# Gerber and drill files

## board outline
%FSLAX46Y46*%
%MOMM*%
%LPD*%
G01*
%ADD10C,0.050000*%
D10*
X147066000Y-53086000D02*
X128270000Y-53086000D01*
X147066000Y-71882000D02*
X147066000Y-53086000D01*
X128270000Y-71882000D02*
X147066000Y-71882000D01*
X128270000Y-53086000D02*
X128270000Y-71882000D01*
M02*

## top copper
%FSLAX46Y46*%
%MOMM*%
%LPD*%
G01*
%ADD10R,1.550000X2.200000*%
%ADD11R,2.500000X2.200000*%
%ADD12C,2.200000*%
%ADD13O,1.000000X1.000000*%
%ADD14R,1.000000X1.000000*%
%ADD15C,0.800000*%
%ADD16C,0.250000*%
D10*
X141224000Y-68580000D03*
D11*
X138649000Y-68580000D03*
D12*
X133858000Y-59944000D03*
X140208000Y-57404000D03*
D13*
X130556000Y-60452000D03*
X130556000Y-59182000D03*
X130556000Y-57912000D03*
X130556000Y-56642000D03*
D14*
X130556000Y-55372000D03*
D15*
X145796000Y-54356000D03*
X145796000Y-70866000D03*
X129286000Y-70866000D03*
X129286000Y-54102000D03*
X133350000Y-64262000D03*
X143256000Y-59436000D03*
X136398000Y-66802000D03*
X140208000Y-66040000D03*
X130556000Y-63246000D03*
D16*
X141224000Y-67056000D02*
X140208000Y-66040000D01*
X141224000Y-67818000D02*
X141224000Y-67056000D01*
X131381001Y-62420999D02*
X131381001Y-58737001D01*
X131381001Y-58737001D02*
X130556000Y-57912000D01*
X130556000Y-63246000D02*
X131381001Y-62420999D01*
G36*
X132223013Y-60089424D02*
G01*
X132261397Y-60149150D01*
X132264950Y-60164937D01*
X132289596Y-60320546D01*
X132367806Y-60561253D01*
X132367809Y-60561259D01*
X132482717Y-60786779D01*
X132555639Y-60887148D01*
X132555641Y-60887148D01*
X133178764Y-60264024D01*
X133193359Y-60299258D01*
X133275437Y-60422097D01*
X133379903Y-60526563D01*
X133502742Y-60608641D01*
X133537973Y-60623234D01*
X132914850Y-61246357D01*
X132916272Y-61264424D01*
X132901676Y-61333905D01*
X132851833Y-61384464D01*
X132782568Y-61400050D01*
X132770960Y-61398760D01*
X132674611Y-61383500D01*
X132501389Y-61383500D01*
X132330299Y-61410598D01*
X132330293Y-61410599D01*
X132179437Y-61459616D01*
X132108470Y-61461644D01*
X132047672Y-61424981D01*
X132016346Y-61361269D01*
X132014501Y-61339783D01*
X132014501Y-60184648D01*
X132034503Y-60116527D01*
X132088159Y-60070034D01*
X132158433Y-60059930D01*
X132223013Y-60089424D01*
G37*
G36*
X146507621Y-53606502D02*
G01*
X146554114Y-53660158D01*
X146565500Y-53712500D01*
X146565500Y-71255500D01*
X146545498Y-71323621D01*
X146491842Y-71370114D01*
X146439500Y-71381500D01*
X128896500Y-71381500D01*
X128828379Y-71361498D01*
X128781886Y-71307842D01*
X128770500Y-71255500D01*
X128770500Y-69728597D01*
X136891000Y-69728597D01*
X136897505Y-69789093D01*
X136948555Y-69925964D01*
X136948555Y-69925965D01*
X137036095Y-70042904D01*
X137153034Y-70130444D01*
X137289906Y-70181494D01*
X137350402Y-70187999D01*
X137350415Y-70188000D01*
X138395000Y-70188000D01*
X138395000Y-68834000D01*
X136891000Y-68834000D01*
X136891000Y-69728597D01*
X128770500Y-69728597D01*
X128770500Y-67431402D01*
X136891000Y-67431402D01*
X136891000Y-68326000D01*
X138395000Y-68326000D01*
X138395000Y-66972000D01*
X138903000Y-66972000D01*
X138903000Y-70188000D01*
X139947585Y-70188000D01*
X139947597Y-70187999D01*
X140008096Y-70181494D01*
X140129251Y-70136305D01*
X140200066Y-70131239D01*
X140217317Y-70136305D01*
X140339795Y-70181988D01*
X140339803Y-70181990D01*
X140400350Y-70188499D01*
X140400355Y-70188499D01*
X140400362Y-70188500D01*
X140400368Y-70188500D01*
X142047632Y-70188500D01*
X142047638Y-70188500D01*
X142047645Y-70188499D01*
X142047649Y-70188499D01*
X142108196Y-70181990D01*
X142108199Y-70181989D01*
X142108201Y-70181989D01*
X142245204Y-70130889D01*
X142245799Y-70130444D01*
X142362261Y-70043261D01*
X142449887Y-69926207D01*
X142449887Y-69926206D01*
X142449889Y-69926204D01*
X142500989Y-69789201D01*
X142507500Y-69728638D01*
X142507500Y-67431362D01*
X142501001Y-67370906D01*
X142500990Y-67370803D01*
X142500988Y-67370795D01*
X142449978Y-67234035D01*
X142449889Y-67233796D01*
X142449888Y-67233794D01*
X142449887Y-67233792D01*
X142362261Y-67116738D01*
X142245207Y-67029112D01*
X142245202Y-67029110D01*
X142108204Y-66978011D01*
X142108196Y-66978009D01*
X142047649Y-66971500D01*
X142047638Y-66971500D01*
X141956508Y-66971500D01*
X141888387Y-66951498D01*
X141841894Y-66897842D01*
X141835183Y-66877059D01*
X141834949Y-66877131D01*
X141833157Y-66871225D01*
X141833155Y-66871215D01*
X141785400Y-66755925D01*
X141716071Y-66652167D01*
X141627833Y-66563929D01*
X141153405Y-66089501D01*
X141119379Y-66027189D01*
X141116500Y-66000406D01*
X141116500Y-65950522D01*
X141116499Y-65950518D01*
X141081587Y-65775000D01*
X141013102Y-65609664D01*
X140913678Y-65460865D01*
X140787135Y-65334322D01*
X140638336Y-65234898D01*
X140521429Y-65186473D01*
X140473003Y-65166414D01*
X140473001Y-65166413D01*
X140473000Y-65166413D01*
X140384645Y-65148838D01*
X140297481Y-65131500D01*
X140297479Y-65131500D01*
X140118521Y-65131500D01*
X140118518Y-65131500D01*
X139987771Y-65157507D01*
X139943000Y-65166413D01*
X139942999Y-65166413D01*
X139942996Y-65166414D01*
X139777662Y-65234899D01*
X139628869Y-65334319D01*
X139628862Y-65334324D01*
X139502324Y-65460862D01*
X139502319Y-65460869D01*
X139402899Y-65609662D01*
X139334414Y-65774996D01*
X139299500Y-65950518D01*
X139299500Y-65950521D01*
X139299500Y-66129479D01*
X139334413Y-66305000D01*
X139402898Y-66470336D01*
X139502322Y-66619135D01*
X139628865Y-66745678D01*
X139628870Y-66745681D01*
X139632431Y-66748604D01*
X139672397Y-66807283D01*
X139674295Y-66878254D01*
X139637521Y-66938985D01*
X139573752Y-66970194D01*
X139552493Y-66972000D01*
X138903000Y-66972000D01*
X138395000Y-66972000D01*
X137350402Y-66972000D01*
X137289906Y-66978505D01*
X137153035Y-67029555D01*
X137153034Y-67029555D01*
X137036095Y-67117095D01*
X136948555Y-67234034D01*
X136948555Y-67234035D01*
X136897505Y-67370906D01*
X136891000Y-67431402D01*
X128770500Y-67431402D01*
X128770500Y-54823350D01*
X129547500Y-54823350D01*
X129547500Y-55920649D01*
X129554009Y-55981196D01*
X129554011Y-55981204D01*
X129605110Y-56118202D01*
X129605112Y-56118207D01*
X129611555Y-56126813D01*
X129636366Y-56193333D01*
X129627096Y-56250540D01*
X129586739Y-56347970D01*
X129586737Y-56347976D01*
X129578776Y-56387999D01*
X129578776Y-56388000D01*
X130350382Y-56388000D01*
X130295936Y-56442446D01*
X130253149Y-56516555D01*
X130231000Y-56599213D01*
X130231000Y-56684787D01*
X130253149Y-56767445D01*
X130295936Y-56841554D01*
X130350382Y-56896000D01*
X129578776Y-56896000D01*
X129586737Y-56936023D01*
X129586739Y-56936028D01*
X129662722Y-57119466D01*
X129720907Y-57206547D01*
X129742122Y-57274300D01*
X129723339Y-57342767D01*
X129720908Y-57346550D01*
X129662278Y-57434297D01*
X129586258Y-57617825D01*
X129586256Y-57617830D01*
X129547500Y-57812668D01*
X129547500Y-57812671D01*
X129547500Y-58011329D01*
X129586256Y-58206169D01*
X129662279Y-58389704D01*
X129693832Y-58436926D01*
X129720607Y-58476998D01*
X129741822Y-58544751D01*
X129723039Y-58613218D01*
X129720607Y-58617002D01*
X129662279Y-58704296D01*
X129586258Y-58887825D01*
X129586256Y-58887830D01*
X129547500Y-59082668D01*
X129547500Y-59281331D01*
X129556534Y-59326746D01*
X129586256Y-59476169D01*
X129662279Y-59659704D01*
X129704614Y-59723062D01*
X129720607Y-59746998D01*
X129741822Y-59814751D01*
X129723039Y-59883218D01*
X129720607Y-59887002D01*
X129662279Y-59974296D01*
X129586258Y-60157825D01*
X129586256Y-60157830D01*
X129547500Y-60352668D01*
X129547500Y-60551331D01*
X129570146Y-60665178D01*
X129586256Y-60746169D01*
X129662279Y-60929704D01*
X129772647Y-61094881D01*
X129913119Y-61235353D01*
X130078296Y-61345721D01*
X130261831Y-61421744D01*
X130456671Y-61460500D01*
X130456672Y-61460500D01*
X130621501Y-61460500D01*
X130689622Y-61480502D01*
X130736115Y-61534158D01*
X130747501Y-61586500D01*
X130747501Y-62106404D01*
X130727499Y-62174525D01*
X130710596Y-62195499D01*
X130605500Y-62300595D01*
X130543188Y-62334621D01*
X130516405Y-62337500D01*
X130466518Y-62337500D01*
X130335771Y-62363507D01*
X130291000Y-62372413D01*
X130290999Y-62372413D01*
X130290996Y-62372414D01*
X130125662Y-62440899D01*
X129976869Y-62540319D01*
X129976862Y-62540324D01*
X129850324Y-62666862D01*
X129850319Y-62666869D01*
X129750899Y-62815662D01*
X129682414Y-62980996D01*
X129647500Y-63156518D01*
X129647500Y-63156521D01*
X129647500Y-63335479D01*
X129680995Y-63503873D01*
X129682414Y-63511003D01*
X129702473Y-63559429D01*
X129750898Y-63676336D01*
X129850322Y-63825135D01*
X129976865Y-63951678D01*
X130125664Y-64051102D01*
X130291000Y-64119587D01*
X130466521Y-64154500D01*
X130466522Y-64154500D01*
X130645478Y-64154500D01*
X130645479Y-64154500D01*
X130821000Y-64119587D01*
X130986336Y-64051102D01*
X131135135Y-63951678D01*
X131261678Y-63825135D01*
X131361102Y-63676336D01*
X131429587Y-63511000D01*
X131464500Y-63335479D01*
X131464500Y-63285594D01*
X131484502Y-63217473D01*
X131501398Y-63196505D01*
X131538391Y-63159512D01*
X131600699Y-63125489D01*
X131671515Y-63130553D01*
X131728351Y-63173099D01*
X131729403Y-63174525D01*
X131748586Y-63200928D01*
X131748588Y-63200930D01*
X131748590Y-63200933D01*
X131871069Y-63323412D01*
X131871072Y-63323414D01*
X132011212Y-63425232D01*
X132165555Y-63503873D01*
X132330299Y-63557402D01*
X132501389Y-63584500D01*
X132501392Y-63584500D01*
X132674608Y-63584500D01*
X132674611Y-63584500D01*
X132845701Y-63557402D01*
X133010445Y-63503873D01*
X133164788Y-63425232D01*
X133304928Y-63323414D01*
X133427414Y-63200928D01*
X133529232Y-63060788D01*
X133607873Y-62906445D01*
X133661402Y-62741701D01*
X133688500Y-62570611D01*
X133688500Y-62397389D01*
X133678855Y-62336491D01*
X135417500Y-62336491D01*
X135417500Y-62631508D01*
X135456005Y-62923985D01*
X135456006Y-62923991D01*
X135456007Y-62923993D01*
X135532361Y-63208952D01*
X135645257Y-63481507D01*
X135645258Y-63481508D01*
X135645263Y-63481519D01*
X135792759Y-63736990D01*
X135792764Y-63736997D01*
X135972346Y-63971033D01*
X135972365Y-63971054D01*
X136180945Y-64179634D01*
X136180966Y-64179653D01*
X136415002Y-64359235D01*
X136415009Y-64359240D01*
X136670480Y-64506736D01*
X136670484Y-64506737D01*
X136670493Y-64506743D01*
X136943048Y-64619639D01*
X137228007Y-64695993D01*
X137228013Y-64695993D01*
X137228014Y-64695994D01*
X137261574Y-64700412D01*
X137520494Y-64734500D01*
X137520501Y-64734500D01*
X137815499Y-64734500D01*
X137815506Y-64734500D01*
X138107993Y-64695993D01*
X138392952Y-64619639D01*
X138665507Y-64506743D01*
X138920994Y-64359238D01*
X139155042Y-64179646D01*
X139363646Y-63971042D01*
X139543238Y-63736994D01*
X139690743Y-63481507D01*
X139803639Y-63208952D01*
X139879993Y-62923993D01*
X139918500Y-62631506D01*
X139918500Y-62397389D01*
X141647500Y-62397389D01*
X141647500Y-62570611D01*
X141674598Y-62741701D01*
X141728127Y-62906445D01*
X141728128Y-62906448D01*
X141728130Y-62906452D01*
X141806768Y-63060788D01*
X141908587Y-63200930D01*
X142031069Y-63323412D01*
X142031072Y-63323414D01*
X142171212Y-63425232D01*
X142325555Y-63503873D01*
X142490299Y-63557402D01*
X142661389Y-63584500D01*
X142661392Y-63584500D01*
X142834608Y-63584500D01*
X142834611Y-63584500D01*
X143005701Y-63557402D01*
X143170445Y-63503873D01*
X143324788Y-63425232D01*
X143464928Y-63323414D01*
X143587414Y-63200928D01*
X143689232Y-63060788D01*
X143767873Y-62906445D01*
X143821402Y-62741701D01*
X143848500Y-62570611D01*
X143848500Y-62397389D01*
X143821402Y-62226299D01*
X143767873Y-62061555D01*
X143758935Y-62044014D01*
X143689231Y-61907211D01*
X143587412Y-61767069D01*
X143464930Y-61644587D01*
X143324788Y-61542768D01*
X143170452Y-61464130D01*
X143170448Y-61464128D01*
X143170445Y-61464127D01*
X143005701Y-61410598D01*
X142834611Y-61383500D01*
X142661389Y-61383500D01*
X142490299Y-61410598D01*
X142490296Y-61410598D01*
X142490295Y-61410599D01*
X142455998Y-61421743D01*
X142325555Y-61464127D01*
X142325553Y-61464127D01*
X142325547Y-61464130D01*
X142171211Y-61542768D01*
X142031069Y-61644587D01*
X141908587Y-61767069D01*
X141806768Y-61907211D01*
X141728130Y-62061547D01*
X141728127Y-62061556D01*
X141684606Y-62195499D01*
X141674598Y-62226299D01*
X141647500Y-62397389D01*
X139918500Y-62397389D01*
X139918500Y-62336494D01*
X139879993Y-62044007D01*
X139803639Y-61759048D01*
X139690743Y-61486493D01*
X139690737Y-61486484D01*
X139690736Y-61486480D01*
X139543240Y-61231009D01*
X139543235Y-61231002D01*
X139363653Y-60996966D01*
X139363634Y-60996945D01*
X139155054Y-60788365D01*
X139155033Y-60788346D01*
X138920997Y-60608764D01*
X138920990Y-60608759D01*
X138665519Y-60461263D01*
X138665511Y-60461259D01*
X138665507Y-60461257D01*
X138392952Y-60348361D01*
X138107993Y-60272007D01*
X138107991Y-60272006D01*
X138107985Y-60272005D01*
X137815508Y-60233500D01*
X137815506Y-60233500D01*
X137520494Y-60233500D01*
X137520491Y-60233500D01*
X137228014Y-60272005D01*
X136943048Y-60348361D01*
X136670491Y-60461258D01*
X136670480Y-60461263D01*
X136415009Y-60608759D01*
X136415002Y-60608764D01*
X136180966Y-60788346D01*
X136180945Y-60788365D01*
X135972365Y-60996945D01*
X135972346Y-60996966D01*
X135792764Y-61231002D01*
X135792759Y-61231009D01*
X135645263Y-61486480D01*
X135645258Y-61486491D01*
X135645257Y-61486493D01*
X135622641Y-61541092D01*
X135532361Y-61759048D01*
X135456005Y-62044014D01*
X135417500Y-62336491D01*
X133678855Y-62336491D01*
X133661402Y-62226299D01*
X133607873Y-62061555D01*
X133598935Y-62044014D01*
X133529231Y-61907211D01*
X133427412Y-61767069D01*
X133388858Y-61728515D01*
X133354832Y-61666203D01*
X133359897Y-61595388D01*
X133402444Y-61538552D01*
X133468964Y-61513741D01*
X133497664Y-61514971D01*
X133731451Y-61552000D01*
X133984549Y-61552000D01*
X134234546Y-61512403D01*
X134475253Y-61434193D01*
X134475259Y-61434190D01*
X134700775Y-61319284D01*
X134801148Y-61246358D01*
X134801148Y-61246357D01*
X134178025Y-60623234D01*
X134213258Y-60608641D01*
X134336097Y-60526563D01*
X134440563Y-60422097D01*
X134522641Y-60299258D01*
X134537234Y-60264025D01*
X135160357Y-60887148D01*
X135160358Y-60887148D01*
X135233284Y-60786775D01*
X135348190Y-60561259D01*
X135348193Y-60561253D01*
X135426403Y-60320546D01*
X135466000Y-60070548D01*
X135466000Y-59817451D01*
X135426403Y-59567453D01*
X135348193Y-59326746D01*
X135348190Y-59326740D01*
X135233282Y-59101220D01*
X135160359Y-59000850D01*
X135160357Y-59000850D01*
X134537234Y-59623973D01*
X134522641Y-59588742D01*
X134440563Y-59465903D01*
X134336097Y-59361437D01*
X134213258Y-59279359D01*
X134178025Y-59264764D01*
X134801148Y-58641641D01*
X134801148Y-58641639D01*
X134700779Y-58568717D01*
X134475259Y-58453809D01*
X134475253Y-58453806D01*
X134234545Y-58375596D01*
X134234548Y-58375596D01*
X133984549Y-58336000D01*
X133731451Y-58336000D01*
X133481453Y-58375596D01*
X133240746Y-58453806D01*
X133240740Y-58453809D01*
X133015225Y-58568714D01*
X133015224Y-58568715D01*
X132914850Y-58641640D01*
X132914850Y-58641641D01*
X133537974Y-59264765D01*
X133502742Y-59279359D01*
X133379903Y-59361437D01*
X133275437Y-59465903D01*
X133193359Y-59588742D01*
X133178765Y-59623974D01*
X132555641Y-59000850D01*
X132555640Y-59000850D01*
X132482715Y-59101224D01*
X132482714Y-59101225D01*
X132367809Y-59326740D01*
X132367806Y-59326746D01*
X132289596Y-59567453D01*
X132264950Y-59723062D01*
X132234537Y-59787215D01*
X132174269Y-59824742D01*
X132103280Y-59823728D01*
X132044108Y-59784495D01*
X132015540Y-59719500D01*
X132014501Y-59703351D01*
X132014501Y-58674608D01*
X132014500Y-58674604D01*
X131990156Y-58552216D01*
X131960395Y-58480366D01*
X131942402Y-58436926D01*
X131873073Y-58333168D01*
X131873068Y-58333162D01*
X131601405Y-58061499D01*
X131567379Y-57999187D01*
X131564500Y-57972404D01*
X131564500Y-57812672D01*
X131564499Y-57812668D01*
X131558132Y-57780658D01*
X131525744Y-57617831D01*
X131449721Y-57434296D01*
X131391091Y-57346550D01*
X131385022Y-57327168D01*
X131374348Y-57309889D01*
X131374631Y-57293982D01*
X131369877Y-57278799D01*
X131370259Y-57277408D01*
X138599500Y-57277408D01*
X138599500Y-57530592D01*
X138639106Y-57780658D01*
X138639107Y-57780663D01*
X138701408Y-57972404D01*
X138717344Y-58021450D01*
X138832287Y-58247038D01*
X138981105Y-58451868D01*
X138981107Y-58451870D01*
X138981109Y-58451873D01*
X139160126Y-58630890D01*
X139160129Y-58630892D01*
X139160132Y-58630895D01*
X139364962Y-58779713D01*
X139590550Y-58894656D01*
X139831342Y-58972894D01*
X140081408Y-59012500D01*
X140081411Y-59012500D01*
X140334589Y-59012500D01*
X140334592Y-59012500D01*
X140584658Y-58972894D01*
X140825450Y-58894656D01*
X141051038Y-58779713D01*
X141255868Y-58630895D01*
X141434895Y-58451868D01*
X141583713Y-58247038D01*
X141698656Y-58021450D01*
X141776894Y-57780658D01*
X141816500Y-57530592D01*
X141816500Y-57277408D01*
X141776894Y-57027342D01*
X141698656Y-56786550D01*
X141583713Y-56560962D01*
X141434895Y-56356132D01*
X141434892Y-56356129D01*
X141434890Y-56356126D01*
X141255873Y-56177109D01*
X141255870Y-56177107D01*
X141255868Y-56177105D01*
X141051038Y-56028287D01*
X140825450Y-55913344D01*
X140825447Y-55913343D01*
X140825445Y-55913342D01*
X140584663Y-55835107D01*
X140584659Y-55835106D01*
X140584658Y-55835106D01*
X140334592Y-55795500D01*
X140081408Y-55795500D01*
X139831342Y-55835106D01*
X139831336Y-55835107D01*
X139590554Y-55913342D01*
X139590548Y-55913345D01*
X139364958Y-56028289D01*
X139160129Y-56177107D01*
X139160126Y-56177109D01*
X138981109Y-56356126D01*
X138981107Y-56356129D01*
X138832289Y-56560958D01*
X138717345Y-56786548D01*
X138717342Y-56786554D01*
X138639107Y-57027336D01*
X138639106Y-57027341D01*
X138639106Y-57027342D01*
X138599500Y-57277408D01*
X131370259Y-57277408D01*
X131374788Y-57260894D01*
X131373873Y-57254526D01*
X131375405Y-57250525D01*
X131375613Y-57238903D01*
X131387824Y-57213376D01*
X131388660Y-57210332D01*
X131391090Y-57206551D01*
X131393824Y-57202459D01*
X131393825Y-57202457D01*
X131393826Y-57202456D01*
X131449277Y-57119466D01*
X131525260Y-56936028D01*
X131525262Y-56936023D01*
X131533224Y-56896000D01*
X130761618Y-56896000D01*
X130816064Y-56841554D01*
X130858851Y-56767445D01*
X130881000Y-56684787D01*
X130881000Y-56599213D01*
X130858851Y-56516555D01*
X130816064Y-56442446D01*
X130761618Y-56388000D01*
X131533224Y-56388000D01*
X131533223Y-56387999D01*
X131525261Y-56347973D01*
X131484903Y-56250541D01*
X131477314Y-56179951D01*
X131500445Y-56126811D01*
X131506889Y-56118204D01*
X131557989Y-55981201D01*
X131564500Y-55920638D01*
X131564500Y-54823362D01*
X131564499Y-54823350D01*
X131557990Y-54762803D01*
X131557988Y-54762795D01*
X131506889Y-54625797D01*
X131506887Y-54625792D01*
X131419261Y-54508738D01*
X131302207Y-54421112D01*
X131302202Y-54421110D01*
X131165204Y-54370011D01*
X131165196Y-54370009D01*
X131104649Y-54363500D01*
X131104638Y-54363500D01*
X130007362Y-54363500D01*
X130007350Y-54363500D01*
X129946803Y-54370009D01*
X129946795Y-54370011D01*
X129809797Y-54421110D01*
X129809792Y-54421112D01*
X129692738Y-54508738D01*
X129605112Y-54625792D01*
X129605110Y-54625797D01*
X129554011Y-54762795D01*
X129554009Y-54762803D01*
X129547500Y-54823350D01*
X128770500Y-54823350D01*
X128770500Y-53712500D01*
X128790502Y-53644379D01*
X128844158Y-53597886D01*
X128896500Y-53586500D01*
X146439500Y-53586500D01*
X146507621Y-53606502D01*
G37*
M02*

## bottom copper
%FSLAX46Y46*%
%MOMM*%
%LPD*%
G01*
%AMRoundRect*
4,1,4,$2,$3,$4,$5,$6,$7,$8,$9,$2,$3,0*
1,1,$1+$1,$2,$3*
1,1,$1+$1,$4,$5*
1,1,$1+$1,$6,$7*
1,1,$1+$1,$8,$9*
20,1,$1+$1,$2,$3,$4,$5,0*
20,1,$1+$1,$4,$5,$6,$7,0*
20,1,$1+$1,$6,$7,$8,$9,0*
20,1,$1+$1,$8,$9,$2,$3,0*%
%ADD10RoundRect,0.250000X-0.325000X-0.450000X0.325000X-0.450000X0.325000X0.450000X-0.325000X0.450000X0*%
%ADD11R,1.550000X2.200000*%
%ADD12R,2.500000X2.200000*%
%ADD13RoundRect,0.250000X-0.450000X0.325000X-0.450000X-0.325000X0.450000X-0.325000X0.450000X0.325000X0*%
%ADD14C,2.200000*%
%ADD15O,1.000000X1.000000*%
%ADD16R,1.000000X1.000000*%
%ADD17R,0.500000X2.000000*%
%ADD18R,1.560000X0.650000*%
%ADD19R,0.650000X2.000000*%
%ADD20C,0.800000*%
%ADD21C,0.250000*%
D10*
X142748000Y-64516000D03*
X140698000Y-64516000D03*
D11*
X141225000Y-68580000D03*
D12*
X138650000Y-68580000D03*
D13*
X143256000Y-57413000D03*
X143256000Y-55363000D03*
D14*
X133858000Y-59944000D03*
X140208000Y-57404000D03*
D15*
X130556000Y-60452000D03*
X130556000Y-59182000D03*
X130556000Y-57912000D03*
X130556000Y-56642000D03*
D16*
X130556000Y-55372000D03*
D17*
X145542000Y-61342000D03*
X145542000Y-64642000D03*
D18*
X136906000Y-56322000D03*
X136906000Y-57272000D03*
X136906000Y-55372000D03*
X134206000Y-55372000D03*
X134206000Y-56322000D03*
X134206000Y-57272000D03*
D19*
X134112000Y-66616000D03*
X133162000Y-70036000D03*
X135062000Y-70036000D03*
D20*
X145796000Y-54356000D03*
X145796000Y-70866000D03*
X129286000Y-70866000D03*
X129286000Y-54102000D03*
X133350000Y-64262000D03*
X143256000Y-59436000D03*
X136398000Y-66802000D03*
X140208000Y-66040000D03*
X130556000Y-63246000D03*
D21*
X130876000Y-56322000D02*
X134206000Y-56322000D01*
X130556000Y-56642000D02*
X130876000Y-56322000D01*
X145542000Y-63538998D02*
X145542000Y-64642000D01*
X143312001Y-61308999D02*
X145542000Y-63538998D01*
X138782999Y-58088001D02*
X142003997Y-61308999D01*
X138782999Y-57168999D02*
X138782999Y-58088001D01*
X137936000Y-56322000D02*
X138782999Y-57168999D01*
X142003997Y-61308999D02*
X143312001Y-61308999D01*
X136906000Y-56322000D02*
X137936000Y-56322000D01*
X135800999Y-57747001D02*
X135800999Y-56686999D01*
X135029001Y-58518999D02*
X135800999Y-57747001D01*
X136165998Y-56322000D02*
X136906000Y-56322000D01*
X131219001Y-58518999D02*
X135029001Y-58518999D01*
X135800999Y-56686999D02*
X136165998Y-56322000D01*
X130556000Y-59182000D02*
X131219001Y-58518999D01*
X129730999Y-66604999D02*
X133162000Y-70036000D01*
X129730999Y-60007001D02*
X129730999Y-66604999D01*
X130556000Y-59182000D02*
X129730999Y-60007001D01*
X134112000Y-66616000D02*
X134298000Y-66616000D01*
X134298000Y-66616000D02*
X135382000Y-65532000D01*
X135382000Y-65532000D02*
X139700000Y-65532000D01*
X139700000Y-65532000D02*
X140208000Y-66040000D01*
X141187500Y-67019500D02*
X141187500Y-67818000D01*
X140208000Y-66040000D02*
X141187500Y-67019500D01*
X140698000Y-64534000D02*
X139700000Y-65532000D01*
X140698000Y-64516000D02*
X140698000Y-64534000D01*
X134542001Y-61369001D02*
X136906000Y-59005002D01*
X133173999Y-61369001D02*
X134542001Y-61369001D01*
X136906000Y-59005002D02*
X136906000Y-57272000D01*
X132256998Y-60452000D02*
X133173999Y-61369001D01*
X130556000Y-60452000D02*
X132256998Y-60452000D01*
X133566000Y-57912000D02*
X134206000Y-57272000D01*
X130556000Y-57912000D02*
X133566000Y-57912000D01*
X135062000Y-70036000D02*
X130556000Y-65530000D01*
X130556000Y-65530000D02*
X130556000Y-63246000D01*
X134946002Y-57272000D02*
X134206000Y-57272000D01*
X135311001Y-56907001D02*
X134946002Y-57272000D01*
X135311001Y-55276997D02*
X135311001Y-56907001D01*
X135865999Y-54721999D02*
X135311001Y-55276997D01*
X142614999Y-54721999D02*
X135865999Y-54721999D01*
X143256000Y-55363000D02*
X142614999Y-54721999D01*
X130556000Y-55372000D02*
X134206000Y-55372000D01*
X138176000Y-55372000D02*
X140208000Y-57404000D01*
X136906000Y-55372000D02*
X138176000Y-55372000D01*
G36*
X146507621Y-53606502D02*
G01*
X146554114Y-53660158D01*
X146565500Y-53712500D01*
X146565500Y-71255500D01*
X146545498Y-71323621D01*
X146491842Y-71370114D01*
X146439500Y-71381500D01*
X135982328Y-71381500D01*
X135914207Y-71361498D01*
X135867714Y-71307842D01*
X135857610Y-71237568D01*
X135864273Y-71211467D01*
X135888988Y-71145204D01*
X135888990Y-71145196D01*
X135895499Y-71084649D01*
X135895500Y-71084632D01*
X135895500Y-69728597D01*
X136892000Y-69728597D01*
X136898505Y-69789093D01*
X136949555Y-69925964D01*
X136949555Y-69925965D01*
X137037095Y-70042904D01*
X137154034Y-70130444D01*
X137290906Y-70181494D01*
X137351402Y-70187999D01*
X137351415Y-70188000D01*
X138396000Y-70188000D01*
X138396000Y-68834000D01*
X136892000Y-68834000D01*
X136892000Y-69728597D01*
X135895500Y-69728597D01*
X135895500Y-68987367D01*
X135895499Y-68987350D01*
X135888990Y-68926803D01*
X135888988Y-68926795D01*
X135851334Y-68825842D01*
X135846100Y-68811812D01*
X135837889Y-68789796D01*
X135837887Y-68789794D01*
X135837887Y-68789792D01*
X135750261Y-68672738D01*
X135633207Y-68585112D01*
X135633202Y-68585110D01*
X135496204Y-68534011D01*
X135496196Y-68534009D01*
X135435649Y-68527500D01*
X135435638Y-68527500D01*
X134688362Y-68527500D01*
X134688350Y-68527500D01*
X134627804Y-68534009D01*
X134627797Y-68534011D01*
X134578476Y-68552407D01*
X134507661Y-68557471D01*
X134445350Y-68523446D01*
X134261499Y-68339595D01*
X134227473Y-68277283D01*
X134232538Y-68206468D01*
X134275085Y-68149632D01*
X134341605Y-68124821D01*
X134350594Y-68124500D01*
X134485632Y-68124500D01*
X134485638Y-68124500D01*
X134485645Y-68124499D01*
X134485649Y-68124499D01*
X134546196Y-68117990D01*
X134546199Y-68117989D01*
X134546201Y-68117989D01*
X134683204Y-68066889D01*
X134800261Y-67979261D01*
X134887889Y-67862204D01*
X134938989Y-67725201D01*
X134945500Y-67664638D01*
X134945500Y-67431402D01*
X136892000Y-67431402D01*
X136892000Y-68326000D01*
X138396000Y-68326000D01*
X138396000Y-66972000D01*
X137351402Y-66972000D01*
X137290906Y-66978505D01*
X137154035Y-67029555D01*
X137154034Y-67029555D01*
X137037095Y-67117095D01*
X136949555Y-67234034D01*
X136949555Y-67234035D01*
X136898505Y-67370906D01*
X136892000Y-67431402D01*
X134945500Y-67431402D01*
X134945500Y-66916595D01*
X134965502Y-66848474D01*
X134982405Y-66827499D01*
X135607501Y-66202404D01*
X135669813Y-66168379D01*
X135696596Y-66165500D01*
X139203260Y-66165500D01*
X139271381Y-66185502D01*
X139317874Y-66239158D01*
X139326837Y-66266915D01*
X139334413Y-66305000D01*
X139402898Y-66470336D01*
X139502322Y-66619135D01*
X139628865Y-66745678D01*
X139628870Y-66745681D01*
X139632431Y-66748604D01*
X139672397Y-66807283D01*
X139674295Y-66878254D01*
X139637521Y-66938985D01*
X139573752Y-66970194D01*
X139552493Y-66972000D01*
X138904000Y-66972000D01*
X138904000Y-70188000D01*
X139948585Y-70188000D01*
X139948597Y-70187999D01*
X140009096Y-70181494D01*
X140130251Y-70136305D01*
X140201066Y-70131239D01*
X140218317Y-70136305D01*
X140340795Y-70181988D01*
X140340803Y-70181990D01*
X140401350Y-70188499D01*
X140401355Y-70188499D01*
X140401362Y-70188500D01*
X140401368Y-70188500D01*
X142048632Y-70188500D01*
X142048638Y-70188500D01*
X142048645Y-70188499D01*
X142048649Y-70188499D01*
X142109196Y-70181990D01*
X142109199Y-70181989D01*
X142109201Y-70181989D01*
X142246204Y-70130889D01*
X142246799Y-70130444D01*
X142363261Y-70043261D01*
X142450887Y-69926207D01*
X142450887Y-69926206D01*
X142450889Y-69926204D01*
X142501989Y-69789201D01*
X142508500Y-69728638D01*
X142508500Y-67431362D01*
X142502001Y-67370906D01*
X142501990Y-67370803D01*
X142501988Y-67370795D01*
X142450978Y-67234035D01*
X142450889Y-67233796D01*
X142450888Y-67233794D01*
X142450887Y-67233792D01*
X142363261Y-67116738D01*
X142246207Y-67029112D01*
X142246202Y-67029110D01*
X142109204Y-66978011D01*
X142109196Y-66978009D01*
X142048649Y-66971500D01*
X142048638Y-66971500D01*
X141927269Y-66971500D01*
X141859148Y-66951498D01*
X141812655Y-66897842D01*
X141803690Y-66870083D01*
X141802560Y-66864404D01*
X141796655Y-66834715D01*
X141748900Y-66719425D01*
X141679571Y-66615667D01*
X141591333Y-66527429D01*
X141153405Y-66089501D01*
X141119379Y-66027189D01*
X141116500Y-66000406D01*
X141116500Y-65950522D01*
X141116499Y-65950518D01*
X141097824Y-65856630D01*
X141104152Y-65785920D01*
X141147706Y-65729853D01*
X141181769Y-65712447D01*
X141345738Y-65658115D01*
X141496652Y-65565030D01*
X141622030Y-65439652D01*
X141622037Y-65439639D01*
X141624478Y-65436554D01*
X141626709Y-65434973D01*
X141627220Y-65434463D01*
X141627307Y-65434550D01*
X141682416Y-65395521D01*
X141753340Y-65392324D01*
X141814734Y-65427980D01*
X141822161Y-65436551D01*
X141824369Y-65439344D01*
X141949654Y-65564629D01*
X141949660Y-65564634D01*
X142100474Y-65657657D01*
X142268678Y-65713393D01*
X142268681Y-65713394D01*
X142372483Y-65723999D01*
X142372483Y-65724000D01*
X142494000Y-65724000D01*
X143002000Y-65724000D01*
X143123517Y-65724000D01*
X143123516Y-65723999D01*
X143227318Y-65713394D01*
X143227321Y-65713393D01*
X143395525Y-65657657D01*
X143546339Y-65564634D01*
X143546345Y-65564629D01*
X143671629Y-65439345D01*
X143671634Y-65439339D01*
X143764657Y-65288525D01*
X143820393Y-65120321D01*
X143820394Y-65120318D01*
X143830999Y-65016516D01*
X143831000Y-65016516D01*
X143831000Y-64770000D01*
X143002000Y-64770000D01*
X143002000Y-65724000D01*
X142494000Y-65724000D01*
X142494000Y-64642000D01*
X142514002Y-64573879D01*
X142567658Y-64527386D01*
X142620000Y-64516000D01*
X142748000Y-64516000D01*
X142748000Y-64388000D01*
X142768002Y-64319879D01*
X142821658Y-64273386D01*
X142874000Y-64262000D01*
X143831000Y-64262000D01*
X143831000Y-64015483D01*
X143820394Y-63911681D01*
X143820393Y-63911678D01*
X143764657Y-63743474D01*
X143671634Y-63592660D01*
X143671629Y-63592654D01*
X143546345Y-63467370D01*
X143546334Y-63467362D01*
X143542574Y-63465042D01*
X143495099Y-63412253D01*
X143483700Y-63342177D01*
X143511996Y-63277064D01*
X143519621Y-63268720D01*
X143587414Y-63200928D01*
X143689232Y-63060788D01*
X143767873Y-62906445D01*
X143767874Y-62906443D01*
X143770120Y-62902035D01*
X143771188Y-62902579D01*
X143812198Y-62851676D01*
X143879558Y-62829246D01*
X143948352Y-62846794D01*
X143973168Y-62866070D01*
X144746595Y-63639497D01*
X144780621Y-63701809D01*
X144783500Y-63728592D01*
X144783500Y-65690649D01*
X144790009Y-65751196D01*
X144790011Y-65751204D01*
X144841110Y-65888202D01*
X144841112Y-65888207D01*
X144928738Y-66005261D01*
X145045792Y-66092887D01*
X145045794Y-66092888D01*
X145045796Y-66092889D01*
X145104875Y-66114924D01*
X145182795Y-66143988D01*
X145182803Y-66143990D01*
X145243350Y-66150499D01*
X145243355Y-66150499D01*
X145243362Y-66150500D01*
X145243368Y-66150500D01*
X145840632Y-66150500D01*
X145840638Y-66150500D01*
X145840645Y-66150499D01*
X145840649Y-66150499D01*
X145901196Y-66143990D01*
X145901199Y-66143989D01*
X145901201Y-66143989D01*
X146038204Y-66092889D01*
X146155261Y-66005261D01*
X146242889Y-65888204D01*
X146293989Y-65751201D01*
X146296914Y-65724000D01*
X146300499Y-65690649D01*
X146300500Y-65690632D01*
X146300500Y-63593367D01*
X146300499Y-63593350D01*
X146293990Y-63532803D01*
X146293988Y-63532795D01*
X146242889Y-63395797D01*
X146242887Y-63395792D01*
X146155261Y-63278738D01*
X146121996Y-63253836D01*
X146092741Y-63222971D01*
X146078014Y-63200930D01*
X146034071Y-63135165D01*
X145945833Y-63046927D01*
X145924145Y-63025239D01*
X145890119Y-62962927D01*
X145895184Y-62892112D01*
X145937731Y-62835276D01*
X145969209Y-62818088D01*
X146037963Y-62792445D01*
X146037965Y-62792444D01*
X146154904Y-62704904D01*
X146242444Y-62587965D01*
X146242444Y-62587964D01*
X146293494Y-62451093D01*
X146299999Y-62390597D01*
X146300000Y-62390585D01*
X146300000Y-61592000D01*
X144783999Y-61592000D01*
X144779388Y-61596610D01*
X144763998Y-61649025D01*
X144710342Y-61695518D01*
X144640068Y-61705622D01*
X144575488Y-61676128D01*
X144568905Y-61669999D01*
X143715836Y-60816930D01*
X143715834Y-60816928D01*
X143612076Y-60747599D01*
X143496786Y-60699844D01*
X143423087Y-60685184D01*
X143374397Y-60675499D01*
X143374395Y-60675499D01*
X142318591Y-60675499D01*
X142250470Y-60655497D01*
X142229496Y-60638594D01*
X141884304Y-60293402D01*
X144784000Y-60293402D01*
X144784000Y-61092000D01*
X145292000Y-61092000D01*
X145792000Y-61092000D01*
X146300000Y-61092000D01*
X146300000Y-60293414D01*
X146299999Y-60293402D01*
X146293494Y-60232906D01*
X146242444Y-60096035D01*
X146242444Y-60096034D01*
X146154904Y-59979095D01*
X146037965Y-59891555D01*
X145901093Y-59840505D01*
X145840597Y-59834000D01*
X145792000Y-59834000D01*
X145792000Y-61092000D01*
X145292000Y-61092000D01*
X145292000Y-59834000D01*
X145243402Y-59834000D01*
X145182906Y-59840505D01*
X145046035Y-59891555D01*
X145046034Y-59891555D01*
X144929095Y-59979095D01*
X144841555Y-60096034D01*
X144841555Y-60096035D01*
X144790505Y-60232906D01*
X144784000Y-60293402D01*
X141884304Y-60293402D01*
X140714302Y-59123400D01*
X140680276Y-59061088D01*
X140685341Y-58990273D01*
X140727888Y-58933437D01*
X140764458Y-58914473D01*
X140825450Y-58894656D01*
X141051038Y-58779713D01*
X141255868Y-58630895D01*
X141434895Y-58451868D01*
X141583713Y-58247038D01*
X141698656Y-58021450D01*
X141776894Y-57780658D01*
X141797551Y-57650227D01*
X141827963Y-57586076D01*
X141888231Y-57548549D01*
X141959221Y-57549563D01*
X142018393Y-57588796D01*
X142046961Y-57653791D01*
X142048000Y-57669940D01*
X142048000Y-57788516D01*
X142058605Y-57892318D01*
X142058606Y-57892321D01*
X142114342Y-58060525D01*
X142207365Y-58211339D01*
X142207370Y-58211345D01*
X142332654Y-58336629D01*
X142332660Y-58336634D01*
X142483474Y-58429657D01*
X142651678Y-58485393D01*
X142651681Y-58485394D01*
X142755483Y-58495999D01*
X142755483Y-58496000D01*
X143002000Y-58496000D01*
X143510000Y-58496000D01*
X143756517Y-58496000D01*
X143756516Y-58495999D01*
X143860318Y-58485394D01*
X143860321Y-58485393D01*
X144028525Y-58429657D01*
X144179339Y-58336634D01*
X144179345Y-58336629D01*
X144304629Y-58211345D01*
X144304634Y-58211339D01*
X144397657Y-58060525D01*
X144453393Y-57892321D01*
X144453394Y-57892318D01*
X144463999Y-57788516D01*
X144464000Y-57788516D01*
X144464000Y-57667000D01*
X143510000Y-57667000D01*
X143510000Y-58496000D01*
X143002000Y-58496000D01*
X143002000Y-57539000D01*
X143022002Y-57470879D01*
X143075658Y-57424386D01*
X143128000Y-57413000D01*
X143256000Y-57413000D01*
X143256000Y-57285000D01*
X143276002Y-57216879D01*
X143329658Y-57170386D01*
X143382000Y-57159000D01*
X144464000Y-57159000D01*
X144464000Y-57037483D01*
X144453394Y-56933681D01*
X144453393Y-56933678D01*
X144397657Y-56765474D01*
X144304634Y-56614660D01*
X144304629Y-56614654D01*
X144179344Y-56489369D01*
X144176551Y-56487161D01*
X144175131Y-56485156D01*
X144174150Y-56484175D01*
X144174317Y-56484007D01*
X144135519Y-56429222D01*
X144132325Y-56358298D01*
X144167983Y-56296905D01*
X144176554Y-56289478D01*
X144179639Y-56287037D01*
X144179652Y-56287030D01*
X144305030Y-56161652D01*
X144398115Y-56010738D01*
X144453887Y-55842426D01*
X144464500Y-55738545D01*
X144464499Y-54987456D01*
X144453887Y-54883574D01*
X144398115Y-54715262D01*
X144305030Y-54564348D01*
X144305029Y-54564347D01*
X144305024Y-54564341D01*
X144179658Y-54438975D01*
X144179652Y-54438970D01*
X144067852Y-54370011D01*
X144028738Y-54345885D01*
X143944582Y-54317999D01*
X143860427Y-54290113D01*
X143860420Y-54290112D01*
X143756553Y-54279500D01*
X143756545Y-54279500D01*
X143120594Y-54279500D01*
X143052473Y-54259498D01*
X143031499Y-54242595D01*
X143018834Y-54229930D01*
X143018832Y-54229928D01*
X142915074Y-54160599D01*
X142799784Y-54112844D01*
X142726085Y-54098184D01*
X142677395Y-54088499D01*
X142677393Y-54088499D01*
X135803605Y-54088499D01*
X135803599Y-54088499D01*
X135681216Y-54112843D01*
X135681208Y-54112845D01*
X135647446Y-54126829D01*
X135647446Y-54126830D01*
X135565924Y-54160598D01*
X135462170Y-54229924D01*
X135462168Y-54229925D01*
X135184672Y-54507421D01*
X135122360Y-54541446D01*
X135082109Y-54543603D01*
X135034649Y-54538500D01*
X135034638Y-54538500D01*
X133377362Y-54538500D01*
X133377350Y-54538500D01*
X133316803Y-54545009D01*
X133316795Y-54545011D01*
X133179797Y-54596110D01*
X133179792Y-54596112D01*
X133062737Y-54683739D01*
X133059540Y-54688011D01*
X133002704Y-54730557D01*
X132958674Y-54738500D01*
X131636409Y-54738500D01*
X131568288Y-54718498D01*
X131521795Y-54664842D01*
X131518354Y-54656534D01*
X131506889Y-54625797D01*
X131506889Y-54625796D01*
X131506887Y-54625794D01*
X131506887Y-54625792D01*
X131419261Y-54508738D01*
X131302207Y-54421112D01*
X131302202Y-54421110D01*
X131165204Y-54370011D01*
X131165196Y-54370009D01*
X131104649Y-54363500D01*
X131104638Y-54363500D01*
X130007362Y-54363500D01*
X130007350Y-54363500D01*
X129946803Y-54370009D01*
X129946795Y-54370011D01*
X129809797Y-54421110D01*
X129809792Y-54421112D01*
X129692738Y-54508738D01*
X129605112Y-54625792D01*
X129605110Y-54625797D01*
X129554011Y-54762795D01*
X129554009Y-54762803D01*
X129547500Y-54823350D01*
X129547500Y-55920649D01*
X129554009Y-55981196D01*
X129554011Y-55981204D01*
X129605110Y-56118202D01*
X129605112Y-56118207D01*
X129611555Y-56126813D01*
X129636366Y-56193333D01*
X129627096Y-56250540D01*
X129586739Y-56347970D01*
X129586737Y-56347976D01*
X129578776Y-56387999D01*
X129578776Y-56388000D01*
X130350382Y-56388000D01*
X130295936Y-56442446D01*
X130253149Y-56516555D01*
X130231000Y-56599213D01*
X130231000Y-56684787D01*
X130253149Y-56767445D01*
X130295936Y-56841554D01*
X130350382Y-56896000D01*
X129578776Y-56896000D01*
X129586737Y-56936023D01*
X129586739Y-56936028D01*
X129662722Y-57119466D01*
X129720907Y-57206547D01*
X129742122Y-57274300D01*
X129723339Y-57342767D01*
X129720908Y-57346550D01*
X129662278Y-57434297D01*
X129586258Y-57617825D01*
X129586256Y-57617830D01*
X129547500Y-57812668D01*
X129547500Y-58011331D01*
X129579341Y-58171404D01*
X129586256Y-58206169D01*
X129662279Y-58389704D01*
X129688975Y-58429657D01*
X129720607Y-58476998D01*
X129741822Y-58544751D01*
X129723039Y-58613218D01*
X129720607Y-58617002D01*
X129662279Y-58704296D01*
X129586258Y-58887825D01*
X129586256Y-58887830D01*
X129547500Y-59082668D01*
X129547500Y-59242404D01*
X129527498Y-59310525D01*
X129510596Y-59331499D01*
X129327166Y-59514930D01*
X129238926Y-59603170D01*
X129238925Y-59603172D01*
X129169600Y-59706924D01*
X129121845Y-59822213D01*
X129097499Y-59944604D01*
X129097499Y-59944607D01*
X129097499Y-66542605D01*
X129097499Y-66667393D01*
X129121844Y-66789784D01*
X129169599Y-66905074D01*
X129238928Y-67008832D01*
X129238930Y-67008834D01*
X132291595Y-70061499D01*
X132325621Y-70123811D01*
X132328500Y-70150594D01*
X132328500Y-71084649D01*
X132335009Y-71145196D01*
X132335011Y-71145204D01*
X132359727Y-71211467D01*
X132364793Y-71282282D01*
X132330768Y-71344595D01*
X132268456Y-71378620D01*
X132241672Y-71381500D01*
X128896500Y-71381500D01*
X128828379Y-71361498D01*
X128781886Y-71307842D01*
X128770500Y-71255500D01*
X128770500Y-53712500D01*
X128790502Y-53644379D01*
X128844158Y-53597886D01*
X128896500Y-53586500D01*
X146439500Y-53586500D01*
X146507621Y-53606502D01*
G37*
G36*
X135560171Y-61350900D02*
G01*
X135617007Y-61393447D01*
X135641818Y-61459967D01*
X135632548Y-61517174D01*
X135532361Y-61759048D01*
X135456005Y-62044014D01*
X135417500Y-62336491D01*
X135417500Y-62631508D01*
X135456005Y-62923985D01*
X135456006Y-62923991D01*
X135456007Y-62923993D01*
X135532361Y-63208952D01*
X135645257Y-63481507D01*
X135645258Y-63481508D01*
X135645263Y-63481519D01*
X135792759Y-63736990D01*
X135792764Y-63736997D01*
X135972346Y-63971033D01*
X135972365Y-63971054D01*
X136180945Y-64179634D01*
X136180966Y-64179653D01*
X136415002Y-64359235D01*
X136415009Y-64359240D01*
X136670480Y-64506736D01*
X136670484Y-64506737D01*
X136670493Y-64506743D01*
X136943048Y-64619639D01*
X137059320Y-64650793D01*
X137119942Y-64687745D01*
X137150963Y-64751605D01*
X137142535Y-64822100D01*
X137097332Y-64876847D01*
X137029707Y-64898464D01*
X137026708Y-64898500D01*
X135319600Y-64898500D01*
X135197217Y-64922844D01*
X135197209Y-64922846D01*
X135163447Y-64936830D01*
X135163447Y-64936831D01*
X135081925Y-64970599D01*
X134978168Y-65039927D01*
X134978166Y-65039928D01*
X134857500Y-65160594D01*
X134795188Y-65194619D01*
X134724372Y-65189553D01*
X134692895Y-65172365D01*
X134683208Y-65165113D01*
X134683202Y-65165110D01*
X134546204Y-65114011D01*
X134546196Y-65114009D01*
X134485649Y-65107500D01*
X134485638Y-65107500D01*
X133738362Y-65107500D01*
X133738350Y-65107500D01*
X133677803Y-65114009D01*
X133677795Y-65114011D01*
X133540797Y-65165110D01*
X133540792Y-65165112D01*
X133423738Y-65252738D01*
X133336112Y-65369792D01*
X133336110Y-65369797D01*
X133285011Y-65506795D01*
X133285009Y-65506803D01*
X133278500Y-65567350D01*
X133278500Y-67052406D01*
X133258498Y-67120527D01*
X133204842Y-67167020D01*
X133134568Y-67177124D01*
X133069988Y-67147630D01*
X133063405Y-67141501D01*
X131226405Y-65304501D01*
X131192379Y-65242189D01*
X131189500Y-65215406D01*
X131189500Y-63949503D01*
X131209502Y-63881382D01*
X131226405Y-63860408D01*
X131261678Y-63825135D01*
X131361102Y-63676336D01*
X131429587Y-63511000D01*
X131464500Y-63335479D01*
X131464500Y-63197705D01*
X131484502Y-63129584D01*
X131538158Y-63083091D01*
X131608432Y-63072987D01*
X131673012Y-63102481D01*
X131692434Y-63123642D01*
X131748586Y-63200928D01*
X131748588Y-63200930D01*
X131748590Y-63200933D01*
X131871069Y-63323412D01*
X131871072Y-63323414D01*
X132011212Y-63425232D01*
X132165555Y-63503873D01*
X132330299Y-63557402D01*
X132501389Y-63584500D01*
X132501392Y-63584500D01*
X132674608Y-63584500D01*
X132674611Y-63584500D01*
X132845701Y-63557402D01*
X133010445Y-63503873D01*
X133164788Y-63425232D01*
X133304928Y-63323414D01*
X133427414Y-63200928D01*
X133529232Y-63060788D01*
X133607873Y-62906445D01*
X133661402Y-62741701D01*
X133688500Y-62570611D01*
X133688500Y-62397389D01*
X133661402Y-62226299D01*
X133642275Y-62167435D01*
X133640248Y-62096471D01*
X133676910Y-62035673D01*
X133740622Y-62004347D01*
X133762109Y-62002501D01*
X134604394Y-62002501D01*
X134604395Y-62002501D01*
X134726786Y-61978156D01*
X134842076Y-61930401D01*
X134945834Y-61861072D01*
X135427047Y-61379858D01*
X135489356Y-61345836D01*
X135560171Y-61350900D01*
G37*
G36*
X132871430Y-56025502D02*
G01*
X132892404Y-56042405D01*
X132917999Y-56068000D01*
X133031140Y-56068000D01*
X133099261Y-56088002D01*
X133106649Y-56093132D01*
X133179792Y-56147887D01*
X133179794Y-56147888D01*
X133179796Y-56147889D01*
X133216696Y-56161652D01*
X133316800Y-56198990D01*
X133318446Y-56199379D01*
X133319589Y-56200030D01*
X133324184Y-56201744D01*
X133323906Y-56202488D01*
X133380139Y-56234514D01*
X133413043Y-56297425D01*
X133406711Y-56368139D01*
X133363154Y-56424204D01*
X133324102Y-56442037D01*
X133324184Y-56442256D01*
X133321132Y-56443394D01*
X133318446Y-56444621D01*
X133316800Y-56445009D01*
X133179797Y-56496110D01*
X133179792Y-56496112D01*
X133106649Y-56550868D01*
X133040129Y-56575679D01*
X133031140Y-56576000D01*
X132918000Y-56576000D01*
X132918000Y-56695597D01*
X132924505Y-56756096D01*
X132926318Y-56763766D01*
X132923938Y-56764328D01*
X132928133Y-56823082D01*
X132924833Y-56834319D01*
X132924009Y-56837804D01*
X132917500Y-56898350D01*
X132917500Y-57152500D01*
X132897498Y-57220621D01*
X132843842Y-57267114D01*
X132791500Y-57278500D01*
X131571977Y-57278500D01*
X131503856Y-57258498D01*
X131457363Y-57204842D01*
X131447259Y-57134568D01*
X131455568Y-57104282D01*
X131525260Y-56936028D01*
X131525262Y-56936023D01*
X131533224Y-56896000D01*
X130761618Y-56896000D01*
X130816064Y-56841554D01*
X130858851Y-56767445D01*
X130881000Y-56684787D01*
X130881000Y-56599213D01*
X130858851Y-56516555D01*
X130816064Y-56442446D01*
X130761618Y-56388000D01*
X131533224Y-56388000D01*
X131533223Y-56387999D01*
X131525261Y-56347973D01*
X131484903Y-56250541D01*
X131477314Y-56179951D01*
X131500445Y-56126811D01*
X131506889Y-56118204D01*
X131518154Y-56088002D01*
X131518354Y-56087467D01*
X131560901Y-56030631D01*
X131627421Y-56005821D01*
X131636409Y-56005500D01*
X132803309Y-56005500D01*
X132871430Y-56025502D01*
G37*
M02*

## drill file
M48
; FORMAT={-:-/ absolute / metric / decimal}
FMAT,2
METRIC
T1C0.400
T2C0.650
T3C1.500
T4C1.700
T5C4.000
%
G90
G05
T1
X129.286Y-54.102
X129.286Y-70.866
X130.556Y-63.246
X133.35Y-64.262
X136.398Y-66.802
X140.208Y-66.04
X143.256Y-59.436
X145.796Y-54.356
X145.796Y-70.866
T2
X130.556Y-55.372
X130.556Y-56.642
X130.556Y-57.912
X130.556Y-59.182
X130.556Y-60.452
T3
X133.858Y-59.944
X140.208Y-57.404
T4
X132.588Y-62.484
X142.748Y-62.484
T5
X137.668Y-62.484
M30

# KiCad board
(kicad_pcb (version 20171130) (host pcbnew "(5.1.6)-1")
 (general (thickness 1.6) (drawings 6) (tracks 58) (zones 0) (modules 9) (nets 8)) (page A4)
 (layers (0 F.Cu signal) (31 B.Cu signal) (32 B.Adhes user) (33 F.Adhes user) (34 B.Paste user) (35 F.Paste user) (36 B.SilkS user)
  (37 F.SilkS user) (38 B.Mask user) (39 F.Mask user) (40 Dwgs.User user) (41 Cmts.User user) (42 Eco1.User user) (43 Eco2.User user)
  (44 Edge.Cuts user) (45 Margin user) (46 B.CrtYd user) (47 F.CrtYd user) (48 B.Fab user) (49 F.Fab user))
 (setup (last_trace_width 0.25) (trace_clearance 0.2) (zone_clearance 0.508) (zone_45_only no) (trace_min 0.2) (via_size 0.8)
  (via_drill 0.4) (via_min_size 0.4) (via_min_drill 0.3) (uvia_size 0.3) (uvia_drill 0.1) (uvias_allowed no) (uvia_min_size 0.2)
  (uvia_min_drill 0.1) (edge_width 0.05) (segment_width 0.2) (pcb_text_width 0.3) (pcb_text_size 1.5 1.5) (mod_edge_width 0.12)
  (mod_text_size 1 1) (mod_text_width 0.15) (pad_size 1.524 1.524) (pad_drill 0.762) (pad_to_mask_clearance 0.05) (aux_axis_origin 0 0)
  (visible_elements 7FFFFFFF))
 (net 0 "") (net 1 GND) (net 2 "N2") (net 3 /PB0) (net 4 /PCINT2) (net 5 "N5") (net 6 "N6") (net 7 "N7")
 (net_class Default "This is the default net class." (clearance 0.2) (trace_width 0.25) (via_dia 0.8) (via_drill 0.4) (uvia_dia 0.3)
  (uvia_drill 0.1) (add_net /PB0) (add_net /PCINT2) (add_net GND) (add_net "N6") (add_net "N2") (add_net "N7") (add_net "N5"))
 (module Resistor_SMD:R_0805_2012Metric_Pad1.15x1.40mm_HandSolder (layer B.Cu) (at 141.723 64.516)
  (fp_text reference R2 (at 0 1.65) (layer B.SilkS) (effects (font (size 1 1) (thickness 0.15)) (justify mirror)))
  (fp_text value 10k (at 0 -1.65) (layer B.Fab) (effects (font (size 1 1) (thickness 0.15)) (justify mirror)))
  (pad 2 smd roundrect (at 1.025 0) (size 1.15 1.4) (layers B.Cu B.Paste B.Mask) (roundrect_rratio 0.217391) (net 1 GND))
  (pad 1 smd roundrect (at -1.025 0) (size 1.15 1.4) (layers B.Cu B.Paste B.Mask) (roundrect_rratio 0.217391) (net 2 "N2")))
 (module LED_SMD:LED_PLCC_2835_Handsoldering (layer B.Cu) (at 139.7 68.58)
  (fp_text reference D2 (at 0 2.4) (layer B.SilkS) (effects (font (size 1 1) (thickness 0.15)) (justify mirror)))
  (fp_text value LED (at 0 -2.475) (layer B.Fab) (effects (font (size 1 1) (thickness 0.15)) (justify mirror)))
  (pad 2 smd rect (at 1.525 0) (size 1.55 2.2) (layers B.Cu B.Paste B.Mask) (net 2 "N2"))
  (pad 1 smd rect (at -1.05 0) (size 2.5 2.2) (layers B.Cu B.Paste B.Mask) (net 1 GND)))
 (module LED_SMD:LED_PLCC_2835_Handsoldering (layer F.Cu) (at 139.699 68.58)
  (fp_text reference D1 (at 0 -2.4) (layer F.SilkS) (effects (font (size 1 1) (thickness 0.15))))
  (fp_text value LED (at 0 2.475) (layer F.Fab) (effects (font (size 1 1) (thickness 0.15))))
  (pad 2 smd rect (at 1.525 0) (size 1.55 2.2) (layers F.Cu F.Paste F.Mask) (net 2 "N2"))
  (pad 1 smd rect (at -1.05 0) (size 2.5 2.2) (layers F.Cu F.Paste F.Mask) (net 1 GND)))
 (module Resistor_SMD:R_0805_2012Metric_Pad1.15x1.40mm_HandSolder (layer B.Cu) (at 143.256 56.388 270)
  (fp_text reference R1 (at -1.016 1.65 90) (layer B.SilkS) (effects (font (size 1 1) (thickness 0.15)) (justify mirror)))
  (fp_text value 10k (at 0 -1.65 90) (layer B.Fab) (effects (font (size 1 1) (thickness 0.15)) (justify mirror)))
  (pad 2 smd roundrect (at 1.025 0 270) (size 1.15 1.4) (layers B.Cu B.Paste B.Mask) (roundrect_rratio 0.217391) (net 1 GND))
  (pad 1 smd roundrect (at -1.025 0 270) (size 1.15 1.4) (layers B.Cu B.Paste B.Mask) (roundrect_rratio 0.217391) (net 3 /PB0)))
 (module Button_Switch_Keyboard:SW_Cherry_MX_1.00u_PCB (layer F.Cu) (at 140.208 57.404)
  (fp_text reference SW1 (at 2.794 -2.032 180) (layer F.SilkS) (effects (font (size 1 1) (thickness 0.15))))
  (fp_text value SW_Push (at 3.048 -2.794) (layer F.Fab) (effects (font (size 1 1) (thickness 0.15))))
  (pad "" np_thru_hole circle (at 2.54 5.08) (size 1.7 1.7) (drill 1.7) (layers *.Cu *.Mask))
  (pad "" np_thru_hole circle (at -7.62 5.08) (size 1.7 1.7) (drill 1.7) (layers *.Cu *.Mask))
  (pad "" np_thru_hole circle (at -2.54 5.08) (size 4 4) (drill 4) (layers *.Cu *.Mask))
  (pad 2 thru_hole circle (at -6.35 2.54) (size 2.2 2.2) (drill 1.5) (layers *.Cu *.Mask) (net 1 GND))
  (pad 1 thru_hole circle (at 0 0) (size 2.2 2.2) (drill 1.5) (layers *.Cu *.Mask) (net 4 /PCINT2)))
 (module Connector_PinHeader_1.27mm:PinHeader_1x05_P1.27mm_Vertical (layer B.Cu) (at 130.556 55.372 180)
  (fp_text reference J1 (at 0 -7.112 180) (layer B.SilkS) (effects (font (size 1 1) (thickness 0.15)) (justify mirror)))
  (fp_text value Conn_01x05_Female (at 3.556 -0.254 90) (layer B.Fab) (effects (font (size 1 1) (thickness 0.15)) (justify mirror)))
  (pad 5 thru_hole oval (at 0 -5.08 180) (size 1 1) (drill 0.65) (layers *.Cu *.Mask) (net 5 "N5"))
  (pad 4 thru_hole oval (at 0 -3.81 180) (size 1 1) (drill 0.65) (layers *.Cu *.Mask) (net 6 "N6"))
  (pad 3 thru_hole oval (at 0 -2.54 180) (size 1 1) (drill 0.65) (layers *.Cu *.Mask) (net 3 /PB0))
  (pad 2 thru_hole oval (at 0 -1.27 180) (size 1 1) (drill 0.65) (layers *.Cu *.Mask) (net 1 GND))
  (pad 1 thru_hole rect (at 0 0 180) (size 1 1) (drill 0.65) (layers *.Cu *.Mask) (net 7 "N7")))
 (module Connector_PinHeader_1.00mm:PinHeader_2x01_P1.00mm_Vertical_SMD (layer B.Cu) (at 145.542 62.992 90)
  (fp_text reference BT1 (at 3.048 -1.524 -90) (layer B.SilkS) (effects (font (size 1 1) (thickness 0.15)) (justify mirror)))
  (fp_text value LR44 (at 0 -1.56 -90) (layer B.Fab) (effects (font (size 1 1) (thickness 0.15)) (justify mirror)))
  (pad 2 smd rect (at 1.65 0 90) (size 2 0.5) (layers B.Cu B.Paste B.Mask) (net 1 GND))
  (pad 1 smd rect (at -1.65 0 90) (size 2 0.5) (layers B.Cu B.Paste B.Mask) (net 6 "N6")))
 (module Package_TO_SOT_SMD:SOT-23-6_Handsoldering (layer B.Cu) (at 135.556 56.322)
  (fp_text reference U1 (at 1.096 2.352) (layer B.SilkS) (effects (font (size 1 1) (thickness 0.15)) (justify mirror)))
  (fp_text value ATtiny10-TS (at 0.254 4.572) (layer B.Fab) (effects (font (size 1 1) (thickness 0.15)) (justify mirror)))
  (pad 5 smd rect (at 1.35 0) (size 1.56 0.65) (layers B.Cu B.Paste B.Mask) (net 6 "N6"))
  (pad 6 smd rect (at 1.35 0.95) (size 1.56 0.65) (layers B.Cu B.Paste B.Mask) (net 5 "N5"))
  (pad 4 smd rect (at 1.35 -0.95) (size 1.56 0.65) (layers B.Cu B.Paste B.Mask) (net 4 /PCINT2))
  (pad 3 smd rect (at -1.35 -0.95) (size 1.56 0.65) (layers B.Cu B.Paste B.Mask) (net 7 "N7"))
  (pad 2 smd rect (at -1.35 0) (size 1.56 0.65) (layers B.Cu B.Paste B.Mask) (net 1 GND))
  (pad 1 smd rect (at -1.35 0.95) (size 1.56 0.65) (layers B.Cu B.Paste B.Mask) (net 3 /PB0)))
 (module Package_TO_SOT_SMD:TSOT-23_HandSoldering (layer B.Cu) (at 134.112 68.326 90)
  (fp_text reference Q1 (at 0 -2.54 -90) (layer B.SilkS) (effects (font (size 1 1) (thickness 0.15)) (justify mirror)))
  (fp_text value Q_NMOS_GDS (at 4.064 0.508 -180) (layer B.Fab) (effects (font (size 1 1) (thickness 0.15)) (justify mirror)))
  (pad 3 smd rect (at 1.71 0 90) (size 2 0.65) (layers B.Cu B.Paste B.Mask) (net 2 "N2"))
  (pad 2 smd rect (at -1.71 -0.95 90) (size 2 0.65) (layers B.Cu B.Paste B.Mask) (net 6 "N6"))
  (pad 1 smd rect (at -1.71 0.95 90) (size 2 0.65) (layers B.Cu B.Paste B.Mask) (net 3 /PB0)))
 (gr_line (start 147.066 53.086) (end 128.27 53.086) (layer Edge.Cuts) (width 0.05))
 (gr_line (start 147.066 71.882) (end 147.066 53.086) (layer Edge.Cuts) (width 0.05))
 (gr_line (start 128.27 71.882) (end 147.066 71.882) (layer Edge.Cuts) (width 0.05))
 (gr_line (start 128.27 53.086) (end 128.27 71.882) (layer Edge.Cuts) (width 0.05))
 (via (at 145.796 54.356) (size 0.8) (drill 0.4) (layers F.Cu B.Cu) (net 1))
 (via (at 145.796 70.866) (size 0.8) (drill 0.4) (layers F.Cu B.Cu) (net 1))
 (segment (start 130.876 56.322) (end 134.206 56.322) (width 0.25) (layer B.Cu) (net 1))
 (segment (start 130.556 56.642) (end 130.876 56.322) (width 0.25) (layer B.Cu) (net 1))
 (via (at 129.286 70.866) (size 0.8) (drill 0.4) (layers F.Cu B.Cu) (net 1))
 (via (at 129.286 54.102) (size 0.8) (drill 0.4) (layers F.Cu B.Cu) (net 1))
 (via (at 133.35 64.262) (size 0.8) (drill 0.4) (layers F.Cu B.Cu) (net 1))
 (via (at 143.256 59.436) (size 0.8) (drill 0.4) (layers F.Cu B.Cu) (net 1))
 (via (at 136.398 66.802) (size 0.8) (drill 0.4) (layers F.Cu B.Cu) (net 1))
 (segment (start 145.542 63.538998) (end 145.542 64.642) (width 0.25) (layer B.Cu) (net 6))
 (segment (start 143.312001 61.308999) (end 145.542 63.538998) (width 0.25) (layer B.Cu) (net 6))
 (segment (start 138.782999 58.088001) (end 142.003997 61.308999) (width 0.25) (layer B.Cu) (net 6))
 (segment (start 138.782999 57.168999) (end 138.782999 58.088001) (width 0.25) (layer B.Cu) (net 6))
 (segment (start 137.936 56.322) (end 138.782999 57.168999) (width 0.25) (layer B.Cu) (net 6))
 (segment (start 142.003997 61.308999) (end 143.312001 61.308999) (width 0.25) (layer B.Cu) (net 6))
 (segment (start 136.906 56.322) (end 137.936 56.322) (width 0.25) (layer B.Cu) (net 6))
 (segment (start 135.800999 57.747001) (end 135.800999 56.686999) (width 0.25) (layer B.Cu) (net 6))
 (segment (start 135.029001 58.518999) (end 135.800999 57.747001) (width 0.25) (layer B.Cu) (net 6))
 (segment (start 136.165998 56.322) (end 136.906 56.322) (width 0.25) (layer B.Cu) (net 6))
 (segment (start 131.219001 58.518999) (end 135.029001 58.518999) (width 0.25) (layer B.Cu) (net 6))
 (segment (start 135.800999 56.686999) (end 136.165998 56.322) (width 0.25) (layer B.Cu) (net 6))
 (segment (start 130.556 59.182) (end 131.219001 58.518999) (width 0.25) (layer B.Cu) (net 6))
 (segment (start 129.730999 66.604999) (end 133.162 70.036) (width 0.25) (layer B.Cu) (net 6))
 (segment (start 129.730999 60.007001) (end 129.730999 66.604999) (width 0.25) (layer B.Cu) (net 6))
 (segment (start 130.556 59.182) (end 129.730999 60.007001) (width 0.25) (layer B.Cu) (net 6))
 (segment (start 134.112 66.616) (end 134.298 66.616) (width 0.25) (layer B.Cu) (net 2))
 (segment (start 134.298 66.616) (end 135.382 65.532) (width 0.25) (layer B.Cu) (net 2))
 (via (at 140.208 66.04) (size 0.8) (drill 0.4) (layers F.Cu B.Cu) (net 2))
 (segment (start 135.382 65.532) (end 139.7 65.532) (width 0.25) (layer B.Cu) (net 2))
 (segment (start 139.7 65.532) (end 140.208 66.04) (width 0.25) (layer B.Cu) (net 2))
 (segment (start 141.224 67.056) (end 140.208 66.04) (width 0.25) (layer F.Cu) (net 2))
 (segment (start 141.224 67.818) (end 141.224 67.056) (width 0.25) (layer F.Cu) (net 2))
 (segment (start 141.1875 67.0195) (end 141.1875 67.818) (width 0.25) (layer B.Cu) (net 2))
 (segment (start 140.208 66.04) (end 141.1875 67.0195) (width 0.25) (layer B.Cu) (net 2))
 (segment (start 140.698 64.534) (end 139.7 65.532) (width 0.25) (layer B.Cu) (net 2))
 (segment (start 140.698 64.516) (end 140.698 64.534) (width 0.25) (layer B.Cu) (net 2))
 (segment (start 134.542001 61.369001) (end 136.906 59.005002) (width 0.25) (layer B.Cu) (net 5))
 (segment (start 133.173999 61.369001) (end 134.542001 61.369001) (width 0.25) (layer B.Cu) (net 5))
 (segment (start 136.906 59.005002) (end 136.906 57.272) (width 0.25) (layer B.Cu) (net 5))
 (segment (start 132.256998 60.452) (end 133.173999 61.369001) (width 0.25) (layer B.Cu) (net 5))
 (segment (start 130.556 60.452) (end 132.256998 60.452) (width 0.25) (layer B.Cu) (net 5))
 (segment (start 133.566 57.912) (end 134.206 57.272) (width 0.25) (layer B.Cu) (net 3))
 (segment (start 130.556 57.912) (end 133.566 57.912) (width 0.25) (layer B.Cu) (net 3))
 (via (at 130.556 63.246) (size 0.8) (drill 0.4) (layers F.Cu B.Cu) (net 3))
 (segment (start 135.062 70.036) (end 130.556 65.53) (width 0.25) (layer B.Cu) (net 3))
 (segment (start 130.556 65.53) (end 130.556 63.246) (width 0.25) (layer B.Cu) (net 3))
 (segment (start 131.381001 62.420999) (end 131.381001 58.737001) (width 0.25) (layer F.Cu) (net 3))
 (segment (start 131.381001 58.737001) (end 130.556 57.912) (width 0.25) (layer F.Cu) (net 3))
 (segment (start 130.556 63.246) (end 131.381001 62.420999) (width 0.25) (layer F.Cu) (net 3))
 (segment (start 134.946002 57.272) (end 134.206 57.272) (width 0.25) (layer B.Cu) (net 3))
 (segment (start 135.311001 56.907001) (end 134.946002 57.272) (width 0.25) (layer B.Cu) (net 3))
 (segment (start 135.311001 55.276997) (end 135.311001 56.907001) (width 0.25) (layer B.Cu) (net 3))
 (segment (start 135.865999 54.721999) (end 135.311001 55.276997) (width 0.25) (layer B.Cu) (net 3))
 (segment (start 142.614999 54.721999) (end 135.865999 54.721999) (width 0.25) (layer B.Cu) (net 3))
 (segment (start 143.256 55.363) (end 142.614999 54.721999) (width 0.25) (layer B.Cu) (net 3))
 (segment (start 130.556 55.372) (end 134.206 55.372) (width 0.25) (layer B.Cu) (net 7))
 (segment (start 138.176 55.372) (end 140.208 57.404) (width 0.25) (layer B.Cu) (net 4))
 (segment (start 136.906 55.372) (end 138.176 55.372) (width 0.25) (layer B.Cu) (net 4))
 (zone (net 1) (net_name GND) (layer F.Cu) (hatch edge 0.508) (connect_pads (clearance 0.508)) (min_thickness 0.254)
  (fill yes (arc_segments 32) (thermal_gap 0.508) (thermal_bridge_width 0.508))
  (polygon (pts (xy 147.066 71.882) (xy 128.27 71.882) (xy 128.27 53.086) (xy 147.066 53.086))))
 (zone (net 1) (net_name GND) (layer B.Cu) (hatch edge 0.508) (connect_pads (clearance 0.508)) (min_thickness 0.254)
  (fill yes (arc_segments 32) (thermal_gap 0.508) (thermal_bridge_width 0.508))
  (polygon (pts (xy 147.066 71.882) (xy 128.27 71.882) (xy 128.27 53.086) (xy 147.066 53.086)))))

